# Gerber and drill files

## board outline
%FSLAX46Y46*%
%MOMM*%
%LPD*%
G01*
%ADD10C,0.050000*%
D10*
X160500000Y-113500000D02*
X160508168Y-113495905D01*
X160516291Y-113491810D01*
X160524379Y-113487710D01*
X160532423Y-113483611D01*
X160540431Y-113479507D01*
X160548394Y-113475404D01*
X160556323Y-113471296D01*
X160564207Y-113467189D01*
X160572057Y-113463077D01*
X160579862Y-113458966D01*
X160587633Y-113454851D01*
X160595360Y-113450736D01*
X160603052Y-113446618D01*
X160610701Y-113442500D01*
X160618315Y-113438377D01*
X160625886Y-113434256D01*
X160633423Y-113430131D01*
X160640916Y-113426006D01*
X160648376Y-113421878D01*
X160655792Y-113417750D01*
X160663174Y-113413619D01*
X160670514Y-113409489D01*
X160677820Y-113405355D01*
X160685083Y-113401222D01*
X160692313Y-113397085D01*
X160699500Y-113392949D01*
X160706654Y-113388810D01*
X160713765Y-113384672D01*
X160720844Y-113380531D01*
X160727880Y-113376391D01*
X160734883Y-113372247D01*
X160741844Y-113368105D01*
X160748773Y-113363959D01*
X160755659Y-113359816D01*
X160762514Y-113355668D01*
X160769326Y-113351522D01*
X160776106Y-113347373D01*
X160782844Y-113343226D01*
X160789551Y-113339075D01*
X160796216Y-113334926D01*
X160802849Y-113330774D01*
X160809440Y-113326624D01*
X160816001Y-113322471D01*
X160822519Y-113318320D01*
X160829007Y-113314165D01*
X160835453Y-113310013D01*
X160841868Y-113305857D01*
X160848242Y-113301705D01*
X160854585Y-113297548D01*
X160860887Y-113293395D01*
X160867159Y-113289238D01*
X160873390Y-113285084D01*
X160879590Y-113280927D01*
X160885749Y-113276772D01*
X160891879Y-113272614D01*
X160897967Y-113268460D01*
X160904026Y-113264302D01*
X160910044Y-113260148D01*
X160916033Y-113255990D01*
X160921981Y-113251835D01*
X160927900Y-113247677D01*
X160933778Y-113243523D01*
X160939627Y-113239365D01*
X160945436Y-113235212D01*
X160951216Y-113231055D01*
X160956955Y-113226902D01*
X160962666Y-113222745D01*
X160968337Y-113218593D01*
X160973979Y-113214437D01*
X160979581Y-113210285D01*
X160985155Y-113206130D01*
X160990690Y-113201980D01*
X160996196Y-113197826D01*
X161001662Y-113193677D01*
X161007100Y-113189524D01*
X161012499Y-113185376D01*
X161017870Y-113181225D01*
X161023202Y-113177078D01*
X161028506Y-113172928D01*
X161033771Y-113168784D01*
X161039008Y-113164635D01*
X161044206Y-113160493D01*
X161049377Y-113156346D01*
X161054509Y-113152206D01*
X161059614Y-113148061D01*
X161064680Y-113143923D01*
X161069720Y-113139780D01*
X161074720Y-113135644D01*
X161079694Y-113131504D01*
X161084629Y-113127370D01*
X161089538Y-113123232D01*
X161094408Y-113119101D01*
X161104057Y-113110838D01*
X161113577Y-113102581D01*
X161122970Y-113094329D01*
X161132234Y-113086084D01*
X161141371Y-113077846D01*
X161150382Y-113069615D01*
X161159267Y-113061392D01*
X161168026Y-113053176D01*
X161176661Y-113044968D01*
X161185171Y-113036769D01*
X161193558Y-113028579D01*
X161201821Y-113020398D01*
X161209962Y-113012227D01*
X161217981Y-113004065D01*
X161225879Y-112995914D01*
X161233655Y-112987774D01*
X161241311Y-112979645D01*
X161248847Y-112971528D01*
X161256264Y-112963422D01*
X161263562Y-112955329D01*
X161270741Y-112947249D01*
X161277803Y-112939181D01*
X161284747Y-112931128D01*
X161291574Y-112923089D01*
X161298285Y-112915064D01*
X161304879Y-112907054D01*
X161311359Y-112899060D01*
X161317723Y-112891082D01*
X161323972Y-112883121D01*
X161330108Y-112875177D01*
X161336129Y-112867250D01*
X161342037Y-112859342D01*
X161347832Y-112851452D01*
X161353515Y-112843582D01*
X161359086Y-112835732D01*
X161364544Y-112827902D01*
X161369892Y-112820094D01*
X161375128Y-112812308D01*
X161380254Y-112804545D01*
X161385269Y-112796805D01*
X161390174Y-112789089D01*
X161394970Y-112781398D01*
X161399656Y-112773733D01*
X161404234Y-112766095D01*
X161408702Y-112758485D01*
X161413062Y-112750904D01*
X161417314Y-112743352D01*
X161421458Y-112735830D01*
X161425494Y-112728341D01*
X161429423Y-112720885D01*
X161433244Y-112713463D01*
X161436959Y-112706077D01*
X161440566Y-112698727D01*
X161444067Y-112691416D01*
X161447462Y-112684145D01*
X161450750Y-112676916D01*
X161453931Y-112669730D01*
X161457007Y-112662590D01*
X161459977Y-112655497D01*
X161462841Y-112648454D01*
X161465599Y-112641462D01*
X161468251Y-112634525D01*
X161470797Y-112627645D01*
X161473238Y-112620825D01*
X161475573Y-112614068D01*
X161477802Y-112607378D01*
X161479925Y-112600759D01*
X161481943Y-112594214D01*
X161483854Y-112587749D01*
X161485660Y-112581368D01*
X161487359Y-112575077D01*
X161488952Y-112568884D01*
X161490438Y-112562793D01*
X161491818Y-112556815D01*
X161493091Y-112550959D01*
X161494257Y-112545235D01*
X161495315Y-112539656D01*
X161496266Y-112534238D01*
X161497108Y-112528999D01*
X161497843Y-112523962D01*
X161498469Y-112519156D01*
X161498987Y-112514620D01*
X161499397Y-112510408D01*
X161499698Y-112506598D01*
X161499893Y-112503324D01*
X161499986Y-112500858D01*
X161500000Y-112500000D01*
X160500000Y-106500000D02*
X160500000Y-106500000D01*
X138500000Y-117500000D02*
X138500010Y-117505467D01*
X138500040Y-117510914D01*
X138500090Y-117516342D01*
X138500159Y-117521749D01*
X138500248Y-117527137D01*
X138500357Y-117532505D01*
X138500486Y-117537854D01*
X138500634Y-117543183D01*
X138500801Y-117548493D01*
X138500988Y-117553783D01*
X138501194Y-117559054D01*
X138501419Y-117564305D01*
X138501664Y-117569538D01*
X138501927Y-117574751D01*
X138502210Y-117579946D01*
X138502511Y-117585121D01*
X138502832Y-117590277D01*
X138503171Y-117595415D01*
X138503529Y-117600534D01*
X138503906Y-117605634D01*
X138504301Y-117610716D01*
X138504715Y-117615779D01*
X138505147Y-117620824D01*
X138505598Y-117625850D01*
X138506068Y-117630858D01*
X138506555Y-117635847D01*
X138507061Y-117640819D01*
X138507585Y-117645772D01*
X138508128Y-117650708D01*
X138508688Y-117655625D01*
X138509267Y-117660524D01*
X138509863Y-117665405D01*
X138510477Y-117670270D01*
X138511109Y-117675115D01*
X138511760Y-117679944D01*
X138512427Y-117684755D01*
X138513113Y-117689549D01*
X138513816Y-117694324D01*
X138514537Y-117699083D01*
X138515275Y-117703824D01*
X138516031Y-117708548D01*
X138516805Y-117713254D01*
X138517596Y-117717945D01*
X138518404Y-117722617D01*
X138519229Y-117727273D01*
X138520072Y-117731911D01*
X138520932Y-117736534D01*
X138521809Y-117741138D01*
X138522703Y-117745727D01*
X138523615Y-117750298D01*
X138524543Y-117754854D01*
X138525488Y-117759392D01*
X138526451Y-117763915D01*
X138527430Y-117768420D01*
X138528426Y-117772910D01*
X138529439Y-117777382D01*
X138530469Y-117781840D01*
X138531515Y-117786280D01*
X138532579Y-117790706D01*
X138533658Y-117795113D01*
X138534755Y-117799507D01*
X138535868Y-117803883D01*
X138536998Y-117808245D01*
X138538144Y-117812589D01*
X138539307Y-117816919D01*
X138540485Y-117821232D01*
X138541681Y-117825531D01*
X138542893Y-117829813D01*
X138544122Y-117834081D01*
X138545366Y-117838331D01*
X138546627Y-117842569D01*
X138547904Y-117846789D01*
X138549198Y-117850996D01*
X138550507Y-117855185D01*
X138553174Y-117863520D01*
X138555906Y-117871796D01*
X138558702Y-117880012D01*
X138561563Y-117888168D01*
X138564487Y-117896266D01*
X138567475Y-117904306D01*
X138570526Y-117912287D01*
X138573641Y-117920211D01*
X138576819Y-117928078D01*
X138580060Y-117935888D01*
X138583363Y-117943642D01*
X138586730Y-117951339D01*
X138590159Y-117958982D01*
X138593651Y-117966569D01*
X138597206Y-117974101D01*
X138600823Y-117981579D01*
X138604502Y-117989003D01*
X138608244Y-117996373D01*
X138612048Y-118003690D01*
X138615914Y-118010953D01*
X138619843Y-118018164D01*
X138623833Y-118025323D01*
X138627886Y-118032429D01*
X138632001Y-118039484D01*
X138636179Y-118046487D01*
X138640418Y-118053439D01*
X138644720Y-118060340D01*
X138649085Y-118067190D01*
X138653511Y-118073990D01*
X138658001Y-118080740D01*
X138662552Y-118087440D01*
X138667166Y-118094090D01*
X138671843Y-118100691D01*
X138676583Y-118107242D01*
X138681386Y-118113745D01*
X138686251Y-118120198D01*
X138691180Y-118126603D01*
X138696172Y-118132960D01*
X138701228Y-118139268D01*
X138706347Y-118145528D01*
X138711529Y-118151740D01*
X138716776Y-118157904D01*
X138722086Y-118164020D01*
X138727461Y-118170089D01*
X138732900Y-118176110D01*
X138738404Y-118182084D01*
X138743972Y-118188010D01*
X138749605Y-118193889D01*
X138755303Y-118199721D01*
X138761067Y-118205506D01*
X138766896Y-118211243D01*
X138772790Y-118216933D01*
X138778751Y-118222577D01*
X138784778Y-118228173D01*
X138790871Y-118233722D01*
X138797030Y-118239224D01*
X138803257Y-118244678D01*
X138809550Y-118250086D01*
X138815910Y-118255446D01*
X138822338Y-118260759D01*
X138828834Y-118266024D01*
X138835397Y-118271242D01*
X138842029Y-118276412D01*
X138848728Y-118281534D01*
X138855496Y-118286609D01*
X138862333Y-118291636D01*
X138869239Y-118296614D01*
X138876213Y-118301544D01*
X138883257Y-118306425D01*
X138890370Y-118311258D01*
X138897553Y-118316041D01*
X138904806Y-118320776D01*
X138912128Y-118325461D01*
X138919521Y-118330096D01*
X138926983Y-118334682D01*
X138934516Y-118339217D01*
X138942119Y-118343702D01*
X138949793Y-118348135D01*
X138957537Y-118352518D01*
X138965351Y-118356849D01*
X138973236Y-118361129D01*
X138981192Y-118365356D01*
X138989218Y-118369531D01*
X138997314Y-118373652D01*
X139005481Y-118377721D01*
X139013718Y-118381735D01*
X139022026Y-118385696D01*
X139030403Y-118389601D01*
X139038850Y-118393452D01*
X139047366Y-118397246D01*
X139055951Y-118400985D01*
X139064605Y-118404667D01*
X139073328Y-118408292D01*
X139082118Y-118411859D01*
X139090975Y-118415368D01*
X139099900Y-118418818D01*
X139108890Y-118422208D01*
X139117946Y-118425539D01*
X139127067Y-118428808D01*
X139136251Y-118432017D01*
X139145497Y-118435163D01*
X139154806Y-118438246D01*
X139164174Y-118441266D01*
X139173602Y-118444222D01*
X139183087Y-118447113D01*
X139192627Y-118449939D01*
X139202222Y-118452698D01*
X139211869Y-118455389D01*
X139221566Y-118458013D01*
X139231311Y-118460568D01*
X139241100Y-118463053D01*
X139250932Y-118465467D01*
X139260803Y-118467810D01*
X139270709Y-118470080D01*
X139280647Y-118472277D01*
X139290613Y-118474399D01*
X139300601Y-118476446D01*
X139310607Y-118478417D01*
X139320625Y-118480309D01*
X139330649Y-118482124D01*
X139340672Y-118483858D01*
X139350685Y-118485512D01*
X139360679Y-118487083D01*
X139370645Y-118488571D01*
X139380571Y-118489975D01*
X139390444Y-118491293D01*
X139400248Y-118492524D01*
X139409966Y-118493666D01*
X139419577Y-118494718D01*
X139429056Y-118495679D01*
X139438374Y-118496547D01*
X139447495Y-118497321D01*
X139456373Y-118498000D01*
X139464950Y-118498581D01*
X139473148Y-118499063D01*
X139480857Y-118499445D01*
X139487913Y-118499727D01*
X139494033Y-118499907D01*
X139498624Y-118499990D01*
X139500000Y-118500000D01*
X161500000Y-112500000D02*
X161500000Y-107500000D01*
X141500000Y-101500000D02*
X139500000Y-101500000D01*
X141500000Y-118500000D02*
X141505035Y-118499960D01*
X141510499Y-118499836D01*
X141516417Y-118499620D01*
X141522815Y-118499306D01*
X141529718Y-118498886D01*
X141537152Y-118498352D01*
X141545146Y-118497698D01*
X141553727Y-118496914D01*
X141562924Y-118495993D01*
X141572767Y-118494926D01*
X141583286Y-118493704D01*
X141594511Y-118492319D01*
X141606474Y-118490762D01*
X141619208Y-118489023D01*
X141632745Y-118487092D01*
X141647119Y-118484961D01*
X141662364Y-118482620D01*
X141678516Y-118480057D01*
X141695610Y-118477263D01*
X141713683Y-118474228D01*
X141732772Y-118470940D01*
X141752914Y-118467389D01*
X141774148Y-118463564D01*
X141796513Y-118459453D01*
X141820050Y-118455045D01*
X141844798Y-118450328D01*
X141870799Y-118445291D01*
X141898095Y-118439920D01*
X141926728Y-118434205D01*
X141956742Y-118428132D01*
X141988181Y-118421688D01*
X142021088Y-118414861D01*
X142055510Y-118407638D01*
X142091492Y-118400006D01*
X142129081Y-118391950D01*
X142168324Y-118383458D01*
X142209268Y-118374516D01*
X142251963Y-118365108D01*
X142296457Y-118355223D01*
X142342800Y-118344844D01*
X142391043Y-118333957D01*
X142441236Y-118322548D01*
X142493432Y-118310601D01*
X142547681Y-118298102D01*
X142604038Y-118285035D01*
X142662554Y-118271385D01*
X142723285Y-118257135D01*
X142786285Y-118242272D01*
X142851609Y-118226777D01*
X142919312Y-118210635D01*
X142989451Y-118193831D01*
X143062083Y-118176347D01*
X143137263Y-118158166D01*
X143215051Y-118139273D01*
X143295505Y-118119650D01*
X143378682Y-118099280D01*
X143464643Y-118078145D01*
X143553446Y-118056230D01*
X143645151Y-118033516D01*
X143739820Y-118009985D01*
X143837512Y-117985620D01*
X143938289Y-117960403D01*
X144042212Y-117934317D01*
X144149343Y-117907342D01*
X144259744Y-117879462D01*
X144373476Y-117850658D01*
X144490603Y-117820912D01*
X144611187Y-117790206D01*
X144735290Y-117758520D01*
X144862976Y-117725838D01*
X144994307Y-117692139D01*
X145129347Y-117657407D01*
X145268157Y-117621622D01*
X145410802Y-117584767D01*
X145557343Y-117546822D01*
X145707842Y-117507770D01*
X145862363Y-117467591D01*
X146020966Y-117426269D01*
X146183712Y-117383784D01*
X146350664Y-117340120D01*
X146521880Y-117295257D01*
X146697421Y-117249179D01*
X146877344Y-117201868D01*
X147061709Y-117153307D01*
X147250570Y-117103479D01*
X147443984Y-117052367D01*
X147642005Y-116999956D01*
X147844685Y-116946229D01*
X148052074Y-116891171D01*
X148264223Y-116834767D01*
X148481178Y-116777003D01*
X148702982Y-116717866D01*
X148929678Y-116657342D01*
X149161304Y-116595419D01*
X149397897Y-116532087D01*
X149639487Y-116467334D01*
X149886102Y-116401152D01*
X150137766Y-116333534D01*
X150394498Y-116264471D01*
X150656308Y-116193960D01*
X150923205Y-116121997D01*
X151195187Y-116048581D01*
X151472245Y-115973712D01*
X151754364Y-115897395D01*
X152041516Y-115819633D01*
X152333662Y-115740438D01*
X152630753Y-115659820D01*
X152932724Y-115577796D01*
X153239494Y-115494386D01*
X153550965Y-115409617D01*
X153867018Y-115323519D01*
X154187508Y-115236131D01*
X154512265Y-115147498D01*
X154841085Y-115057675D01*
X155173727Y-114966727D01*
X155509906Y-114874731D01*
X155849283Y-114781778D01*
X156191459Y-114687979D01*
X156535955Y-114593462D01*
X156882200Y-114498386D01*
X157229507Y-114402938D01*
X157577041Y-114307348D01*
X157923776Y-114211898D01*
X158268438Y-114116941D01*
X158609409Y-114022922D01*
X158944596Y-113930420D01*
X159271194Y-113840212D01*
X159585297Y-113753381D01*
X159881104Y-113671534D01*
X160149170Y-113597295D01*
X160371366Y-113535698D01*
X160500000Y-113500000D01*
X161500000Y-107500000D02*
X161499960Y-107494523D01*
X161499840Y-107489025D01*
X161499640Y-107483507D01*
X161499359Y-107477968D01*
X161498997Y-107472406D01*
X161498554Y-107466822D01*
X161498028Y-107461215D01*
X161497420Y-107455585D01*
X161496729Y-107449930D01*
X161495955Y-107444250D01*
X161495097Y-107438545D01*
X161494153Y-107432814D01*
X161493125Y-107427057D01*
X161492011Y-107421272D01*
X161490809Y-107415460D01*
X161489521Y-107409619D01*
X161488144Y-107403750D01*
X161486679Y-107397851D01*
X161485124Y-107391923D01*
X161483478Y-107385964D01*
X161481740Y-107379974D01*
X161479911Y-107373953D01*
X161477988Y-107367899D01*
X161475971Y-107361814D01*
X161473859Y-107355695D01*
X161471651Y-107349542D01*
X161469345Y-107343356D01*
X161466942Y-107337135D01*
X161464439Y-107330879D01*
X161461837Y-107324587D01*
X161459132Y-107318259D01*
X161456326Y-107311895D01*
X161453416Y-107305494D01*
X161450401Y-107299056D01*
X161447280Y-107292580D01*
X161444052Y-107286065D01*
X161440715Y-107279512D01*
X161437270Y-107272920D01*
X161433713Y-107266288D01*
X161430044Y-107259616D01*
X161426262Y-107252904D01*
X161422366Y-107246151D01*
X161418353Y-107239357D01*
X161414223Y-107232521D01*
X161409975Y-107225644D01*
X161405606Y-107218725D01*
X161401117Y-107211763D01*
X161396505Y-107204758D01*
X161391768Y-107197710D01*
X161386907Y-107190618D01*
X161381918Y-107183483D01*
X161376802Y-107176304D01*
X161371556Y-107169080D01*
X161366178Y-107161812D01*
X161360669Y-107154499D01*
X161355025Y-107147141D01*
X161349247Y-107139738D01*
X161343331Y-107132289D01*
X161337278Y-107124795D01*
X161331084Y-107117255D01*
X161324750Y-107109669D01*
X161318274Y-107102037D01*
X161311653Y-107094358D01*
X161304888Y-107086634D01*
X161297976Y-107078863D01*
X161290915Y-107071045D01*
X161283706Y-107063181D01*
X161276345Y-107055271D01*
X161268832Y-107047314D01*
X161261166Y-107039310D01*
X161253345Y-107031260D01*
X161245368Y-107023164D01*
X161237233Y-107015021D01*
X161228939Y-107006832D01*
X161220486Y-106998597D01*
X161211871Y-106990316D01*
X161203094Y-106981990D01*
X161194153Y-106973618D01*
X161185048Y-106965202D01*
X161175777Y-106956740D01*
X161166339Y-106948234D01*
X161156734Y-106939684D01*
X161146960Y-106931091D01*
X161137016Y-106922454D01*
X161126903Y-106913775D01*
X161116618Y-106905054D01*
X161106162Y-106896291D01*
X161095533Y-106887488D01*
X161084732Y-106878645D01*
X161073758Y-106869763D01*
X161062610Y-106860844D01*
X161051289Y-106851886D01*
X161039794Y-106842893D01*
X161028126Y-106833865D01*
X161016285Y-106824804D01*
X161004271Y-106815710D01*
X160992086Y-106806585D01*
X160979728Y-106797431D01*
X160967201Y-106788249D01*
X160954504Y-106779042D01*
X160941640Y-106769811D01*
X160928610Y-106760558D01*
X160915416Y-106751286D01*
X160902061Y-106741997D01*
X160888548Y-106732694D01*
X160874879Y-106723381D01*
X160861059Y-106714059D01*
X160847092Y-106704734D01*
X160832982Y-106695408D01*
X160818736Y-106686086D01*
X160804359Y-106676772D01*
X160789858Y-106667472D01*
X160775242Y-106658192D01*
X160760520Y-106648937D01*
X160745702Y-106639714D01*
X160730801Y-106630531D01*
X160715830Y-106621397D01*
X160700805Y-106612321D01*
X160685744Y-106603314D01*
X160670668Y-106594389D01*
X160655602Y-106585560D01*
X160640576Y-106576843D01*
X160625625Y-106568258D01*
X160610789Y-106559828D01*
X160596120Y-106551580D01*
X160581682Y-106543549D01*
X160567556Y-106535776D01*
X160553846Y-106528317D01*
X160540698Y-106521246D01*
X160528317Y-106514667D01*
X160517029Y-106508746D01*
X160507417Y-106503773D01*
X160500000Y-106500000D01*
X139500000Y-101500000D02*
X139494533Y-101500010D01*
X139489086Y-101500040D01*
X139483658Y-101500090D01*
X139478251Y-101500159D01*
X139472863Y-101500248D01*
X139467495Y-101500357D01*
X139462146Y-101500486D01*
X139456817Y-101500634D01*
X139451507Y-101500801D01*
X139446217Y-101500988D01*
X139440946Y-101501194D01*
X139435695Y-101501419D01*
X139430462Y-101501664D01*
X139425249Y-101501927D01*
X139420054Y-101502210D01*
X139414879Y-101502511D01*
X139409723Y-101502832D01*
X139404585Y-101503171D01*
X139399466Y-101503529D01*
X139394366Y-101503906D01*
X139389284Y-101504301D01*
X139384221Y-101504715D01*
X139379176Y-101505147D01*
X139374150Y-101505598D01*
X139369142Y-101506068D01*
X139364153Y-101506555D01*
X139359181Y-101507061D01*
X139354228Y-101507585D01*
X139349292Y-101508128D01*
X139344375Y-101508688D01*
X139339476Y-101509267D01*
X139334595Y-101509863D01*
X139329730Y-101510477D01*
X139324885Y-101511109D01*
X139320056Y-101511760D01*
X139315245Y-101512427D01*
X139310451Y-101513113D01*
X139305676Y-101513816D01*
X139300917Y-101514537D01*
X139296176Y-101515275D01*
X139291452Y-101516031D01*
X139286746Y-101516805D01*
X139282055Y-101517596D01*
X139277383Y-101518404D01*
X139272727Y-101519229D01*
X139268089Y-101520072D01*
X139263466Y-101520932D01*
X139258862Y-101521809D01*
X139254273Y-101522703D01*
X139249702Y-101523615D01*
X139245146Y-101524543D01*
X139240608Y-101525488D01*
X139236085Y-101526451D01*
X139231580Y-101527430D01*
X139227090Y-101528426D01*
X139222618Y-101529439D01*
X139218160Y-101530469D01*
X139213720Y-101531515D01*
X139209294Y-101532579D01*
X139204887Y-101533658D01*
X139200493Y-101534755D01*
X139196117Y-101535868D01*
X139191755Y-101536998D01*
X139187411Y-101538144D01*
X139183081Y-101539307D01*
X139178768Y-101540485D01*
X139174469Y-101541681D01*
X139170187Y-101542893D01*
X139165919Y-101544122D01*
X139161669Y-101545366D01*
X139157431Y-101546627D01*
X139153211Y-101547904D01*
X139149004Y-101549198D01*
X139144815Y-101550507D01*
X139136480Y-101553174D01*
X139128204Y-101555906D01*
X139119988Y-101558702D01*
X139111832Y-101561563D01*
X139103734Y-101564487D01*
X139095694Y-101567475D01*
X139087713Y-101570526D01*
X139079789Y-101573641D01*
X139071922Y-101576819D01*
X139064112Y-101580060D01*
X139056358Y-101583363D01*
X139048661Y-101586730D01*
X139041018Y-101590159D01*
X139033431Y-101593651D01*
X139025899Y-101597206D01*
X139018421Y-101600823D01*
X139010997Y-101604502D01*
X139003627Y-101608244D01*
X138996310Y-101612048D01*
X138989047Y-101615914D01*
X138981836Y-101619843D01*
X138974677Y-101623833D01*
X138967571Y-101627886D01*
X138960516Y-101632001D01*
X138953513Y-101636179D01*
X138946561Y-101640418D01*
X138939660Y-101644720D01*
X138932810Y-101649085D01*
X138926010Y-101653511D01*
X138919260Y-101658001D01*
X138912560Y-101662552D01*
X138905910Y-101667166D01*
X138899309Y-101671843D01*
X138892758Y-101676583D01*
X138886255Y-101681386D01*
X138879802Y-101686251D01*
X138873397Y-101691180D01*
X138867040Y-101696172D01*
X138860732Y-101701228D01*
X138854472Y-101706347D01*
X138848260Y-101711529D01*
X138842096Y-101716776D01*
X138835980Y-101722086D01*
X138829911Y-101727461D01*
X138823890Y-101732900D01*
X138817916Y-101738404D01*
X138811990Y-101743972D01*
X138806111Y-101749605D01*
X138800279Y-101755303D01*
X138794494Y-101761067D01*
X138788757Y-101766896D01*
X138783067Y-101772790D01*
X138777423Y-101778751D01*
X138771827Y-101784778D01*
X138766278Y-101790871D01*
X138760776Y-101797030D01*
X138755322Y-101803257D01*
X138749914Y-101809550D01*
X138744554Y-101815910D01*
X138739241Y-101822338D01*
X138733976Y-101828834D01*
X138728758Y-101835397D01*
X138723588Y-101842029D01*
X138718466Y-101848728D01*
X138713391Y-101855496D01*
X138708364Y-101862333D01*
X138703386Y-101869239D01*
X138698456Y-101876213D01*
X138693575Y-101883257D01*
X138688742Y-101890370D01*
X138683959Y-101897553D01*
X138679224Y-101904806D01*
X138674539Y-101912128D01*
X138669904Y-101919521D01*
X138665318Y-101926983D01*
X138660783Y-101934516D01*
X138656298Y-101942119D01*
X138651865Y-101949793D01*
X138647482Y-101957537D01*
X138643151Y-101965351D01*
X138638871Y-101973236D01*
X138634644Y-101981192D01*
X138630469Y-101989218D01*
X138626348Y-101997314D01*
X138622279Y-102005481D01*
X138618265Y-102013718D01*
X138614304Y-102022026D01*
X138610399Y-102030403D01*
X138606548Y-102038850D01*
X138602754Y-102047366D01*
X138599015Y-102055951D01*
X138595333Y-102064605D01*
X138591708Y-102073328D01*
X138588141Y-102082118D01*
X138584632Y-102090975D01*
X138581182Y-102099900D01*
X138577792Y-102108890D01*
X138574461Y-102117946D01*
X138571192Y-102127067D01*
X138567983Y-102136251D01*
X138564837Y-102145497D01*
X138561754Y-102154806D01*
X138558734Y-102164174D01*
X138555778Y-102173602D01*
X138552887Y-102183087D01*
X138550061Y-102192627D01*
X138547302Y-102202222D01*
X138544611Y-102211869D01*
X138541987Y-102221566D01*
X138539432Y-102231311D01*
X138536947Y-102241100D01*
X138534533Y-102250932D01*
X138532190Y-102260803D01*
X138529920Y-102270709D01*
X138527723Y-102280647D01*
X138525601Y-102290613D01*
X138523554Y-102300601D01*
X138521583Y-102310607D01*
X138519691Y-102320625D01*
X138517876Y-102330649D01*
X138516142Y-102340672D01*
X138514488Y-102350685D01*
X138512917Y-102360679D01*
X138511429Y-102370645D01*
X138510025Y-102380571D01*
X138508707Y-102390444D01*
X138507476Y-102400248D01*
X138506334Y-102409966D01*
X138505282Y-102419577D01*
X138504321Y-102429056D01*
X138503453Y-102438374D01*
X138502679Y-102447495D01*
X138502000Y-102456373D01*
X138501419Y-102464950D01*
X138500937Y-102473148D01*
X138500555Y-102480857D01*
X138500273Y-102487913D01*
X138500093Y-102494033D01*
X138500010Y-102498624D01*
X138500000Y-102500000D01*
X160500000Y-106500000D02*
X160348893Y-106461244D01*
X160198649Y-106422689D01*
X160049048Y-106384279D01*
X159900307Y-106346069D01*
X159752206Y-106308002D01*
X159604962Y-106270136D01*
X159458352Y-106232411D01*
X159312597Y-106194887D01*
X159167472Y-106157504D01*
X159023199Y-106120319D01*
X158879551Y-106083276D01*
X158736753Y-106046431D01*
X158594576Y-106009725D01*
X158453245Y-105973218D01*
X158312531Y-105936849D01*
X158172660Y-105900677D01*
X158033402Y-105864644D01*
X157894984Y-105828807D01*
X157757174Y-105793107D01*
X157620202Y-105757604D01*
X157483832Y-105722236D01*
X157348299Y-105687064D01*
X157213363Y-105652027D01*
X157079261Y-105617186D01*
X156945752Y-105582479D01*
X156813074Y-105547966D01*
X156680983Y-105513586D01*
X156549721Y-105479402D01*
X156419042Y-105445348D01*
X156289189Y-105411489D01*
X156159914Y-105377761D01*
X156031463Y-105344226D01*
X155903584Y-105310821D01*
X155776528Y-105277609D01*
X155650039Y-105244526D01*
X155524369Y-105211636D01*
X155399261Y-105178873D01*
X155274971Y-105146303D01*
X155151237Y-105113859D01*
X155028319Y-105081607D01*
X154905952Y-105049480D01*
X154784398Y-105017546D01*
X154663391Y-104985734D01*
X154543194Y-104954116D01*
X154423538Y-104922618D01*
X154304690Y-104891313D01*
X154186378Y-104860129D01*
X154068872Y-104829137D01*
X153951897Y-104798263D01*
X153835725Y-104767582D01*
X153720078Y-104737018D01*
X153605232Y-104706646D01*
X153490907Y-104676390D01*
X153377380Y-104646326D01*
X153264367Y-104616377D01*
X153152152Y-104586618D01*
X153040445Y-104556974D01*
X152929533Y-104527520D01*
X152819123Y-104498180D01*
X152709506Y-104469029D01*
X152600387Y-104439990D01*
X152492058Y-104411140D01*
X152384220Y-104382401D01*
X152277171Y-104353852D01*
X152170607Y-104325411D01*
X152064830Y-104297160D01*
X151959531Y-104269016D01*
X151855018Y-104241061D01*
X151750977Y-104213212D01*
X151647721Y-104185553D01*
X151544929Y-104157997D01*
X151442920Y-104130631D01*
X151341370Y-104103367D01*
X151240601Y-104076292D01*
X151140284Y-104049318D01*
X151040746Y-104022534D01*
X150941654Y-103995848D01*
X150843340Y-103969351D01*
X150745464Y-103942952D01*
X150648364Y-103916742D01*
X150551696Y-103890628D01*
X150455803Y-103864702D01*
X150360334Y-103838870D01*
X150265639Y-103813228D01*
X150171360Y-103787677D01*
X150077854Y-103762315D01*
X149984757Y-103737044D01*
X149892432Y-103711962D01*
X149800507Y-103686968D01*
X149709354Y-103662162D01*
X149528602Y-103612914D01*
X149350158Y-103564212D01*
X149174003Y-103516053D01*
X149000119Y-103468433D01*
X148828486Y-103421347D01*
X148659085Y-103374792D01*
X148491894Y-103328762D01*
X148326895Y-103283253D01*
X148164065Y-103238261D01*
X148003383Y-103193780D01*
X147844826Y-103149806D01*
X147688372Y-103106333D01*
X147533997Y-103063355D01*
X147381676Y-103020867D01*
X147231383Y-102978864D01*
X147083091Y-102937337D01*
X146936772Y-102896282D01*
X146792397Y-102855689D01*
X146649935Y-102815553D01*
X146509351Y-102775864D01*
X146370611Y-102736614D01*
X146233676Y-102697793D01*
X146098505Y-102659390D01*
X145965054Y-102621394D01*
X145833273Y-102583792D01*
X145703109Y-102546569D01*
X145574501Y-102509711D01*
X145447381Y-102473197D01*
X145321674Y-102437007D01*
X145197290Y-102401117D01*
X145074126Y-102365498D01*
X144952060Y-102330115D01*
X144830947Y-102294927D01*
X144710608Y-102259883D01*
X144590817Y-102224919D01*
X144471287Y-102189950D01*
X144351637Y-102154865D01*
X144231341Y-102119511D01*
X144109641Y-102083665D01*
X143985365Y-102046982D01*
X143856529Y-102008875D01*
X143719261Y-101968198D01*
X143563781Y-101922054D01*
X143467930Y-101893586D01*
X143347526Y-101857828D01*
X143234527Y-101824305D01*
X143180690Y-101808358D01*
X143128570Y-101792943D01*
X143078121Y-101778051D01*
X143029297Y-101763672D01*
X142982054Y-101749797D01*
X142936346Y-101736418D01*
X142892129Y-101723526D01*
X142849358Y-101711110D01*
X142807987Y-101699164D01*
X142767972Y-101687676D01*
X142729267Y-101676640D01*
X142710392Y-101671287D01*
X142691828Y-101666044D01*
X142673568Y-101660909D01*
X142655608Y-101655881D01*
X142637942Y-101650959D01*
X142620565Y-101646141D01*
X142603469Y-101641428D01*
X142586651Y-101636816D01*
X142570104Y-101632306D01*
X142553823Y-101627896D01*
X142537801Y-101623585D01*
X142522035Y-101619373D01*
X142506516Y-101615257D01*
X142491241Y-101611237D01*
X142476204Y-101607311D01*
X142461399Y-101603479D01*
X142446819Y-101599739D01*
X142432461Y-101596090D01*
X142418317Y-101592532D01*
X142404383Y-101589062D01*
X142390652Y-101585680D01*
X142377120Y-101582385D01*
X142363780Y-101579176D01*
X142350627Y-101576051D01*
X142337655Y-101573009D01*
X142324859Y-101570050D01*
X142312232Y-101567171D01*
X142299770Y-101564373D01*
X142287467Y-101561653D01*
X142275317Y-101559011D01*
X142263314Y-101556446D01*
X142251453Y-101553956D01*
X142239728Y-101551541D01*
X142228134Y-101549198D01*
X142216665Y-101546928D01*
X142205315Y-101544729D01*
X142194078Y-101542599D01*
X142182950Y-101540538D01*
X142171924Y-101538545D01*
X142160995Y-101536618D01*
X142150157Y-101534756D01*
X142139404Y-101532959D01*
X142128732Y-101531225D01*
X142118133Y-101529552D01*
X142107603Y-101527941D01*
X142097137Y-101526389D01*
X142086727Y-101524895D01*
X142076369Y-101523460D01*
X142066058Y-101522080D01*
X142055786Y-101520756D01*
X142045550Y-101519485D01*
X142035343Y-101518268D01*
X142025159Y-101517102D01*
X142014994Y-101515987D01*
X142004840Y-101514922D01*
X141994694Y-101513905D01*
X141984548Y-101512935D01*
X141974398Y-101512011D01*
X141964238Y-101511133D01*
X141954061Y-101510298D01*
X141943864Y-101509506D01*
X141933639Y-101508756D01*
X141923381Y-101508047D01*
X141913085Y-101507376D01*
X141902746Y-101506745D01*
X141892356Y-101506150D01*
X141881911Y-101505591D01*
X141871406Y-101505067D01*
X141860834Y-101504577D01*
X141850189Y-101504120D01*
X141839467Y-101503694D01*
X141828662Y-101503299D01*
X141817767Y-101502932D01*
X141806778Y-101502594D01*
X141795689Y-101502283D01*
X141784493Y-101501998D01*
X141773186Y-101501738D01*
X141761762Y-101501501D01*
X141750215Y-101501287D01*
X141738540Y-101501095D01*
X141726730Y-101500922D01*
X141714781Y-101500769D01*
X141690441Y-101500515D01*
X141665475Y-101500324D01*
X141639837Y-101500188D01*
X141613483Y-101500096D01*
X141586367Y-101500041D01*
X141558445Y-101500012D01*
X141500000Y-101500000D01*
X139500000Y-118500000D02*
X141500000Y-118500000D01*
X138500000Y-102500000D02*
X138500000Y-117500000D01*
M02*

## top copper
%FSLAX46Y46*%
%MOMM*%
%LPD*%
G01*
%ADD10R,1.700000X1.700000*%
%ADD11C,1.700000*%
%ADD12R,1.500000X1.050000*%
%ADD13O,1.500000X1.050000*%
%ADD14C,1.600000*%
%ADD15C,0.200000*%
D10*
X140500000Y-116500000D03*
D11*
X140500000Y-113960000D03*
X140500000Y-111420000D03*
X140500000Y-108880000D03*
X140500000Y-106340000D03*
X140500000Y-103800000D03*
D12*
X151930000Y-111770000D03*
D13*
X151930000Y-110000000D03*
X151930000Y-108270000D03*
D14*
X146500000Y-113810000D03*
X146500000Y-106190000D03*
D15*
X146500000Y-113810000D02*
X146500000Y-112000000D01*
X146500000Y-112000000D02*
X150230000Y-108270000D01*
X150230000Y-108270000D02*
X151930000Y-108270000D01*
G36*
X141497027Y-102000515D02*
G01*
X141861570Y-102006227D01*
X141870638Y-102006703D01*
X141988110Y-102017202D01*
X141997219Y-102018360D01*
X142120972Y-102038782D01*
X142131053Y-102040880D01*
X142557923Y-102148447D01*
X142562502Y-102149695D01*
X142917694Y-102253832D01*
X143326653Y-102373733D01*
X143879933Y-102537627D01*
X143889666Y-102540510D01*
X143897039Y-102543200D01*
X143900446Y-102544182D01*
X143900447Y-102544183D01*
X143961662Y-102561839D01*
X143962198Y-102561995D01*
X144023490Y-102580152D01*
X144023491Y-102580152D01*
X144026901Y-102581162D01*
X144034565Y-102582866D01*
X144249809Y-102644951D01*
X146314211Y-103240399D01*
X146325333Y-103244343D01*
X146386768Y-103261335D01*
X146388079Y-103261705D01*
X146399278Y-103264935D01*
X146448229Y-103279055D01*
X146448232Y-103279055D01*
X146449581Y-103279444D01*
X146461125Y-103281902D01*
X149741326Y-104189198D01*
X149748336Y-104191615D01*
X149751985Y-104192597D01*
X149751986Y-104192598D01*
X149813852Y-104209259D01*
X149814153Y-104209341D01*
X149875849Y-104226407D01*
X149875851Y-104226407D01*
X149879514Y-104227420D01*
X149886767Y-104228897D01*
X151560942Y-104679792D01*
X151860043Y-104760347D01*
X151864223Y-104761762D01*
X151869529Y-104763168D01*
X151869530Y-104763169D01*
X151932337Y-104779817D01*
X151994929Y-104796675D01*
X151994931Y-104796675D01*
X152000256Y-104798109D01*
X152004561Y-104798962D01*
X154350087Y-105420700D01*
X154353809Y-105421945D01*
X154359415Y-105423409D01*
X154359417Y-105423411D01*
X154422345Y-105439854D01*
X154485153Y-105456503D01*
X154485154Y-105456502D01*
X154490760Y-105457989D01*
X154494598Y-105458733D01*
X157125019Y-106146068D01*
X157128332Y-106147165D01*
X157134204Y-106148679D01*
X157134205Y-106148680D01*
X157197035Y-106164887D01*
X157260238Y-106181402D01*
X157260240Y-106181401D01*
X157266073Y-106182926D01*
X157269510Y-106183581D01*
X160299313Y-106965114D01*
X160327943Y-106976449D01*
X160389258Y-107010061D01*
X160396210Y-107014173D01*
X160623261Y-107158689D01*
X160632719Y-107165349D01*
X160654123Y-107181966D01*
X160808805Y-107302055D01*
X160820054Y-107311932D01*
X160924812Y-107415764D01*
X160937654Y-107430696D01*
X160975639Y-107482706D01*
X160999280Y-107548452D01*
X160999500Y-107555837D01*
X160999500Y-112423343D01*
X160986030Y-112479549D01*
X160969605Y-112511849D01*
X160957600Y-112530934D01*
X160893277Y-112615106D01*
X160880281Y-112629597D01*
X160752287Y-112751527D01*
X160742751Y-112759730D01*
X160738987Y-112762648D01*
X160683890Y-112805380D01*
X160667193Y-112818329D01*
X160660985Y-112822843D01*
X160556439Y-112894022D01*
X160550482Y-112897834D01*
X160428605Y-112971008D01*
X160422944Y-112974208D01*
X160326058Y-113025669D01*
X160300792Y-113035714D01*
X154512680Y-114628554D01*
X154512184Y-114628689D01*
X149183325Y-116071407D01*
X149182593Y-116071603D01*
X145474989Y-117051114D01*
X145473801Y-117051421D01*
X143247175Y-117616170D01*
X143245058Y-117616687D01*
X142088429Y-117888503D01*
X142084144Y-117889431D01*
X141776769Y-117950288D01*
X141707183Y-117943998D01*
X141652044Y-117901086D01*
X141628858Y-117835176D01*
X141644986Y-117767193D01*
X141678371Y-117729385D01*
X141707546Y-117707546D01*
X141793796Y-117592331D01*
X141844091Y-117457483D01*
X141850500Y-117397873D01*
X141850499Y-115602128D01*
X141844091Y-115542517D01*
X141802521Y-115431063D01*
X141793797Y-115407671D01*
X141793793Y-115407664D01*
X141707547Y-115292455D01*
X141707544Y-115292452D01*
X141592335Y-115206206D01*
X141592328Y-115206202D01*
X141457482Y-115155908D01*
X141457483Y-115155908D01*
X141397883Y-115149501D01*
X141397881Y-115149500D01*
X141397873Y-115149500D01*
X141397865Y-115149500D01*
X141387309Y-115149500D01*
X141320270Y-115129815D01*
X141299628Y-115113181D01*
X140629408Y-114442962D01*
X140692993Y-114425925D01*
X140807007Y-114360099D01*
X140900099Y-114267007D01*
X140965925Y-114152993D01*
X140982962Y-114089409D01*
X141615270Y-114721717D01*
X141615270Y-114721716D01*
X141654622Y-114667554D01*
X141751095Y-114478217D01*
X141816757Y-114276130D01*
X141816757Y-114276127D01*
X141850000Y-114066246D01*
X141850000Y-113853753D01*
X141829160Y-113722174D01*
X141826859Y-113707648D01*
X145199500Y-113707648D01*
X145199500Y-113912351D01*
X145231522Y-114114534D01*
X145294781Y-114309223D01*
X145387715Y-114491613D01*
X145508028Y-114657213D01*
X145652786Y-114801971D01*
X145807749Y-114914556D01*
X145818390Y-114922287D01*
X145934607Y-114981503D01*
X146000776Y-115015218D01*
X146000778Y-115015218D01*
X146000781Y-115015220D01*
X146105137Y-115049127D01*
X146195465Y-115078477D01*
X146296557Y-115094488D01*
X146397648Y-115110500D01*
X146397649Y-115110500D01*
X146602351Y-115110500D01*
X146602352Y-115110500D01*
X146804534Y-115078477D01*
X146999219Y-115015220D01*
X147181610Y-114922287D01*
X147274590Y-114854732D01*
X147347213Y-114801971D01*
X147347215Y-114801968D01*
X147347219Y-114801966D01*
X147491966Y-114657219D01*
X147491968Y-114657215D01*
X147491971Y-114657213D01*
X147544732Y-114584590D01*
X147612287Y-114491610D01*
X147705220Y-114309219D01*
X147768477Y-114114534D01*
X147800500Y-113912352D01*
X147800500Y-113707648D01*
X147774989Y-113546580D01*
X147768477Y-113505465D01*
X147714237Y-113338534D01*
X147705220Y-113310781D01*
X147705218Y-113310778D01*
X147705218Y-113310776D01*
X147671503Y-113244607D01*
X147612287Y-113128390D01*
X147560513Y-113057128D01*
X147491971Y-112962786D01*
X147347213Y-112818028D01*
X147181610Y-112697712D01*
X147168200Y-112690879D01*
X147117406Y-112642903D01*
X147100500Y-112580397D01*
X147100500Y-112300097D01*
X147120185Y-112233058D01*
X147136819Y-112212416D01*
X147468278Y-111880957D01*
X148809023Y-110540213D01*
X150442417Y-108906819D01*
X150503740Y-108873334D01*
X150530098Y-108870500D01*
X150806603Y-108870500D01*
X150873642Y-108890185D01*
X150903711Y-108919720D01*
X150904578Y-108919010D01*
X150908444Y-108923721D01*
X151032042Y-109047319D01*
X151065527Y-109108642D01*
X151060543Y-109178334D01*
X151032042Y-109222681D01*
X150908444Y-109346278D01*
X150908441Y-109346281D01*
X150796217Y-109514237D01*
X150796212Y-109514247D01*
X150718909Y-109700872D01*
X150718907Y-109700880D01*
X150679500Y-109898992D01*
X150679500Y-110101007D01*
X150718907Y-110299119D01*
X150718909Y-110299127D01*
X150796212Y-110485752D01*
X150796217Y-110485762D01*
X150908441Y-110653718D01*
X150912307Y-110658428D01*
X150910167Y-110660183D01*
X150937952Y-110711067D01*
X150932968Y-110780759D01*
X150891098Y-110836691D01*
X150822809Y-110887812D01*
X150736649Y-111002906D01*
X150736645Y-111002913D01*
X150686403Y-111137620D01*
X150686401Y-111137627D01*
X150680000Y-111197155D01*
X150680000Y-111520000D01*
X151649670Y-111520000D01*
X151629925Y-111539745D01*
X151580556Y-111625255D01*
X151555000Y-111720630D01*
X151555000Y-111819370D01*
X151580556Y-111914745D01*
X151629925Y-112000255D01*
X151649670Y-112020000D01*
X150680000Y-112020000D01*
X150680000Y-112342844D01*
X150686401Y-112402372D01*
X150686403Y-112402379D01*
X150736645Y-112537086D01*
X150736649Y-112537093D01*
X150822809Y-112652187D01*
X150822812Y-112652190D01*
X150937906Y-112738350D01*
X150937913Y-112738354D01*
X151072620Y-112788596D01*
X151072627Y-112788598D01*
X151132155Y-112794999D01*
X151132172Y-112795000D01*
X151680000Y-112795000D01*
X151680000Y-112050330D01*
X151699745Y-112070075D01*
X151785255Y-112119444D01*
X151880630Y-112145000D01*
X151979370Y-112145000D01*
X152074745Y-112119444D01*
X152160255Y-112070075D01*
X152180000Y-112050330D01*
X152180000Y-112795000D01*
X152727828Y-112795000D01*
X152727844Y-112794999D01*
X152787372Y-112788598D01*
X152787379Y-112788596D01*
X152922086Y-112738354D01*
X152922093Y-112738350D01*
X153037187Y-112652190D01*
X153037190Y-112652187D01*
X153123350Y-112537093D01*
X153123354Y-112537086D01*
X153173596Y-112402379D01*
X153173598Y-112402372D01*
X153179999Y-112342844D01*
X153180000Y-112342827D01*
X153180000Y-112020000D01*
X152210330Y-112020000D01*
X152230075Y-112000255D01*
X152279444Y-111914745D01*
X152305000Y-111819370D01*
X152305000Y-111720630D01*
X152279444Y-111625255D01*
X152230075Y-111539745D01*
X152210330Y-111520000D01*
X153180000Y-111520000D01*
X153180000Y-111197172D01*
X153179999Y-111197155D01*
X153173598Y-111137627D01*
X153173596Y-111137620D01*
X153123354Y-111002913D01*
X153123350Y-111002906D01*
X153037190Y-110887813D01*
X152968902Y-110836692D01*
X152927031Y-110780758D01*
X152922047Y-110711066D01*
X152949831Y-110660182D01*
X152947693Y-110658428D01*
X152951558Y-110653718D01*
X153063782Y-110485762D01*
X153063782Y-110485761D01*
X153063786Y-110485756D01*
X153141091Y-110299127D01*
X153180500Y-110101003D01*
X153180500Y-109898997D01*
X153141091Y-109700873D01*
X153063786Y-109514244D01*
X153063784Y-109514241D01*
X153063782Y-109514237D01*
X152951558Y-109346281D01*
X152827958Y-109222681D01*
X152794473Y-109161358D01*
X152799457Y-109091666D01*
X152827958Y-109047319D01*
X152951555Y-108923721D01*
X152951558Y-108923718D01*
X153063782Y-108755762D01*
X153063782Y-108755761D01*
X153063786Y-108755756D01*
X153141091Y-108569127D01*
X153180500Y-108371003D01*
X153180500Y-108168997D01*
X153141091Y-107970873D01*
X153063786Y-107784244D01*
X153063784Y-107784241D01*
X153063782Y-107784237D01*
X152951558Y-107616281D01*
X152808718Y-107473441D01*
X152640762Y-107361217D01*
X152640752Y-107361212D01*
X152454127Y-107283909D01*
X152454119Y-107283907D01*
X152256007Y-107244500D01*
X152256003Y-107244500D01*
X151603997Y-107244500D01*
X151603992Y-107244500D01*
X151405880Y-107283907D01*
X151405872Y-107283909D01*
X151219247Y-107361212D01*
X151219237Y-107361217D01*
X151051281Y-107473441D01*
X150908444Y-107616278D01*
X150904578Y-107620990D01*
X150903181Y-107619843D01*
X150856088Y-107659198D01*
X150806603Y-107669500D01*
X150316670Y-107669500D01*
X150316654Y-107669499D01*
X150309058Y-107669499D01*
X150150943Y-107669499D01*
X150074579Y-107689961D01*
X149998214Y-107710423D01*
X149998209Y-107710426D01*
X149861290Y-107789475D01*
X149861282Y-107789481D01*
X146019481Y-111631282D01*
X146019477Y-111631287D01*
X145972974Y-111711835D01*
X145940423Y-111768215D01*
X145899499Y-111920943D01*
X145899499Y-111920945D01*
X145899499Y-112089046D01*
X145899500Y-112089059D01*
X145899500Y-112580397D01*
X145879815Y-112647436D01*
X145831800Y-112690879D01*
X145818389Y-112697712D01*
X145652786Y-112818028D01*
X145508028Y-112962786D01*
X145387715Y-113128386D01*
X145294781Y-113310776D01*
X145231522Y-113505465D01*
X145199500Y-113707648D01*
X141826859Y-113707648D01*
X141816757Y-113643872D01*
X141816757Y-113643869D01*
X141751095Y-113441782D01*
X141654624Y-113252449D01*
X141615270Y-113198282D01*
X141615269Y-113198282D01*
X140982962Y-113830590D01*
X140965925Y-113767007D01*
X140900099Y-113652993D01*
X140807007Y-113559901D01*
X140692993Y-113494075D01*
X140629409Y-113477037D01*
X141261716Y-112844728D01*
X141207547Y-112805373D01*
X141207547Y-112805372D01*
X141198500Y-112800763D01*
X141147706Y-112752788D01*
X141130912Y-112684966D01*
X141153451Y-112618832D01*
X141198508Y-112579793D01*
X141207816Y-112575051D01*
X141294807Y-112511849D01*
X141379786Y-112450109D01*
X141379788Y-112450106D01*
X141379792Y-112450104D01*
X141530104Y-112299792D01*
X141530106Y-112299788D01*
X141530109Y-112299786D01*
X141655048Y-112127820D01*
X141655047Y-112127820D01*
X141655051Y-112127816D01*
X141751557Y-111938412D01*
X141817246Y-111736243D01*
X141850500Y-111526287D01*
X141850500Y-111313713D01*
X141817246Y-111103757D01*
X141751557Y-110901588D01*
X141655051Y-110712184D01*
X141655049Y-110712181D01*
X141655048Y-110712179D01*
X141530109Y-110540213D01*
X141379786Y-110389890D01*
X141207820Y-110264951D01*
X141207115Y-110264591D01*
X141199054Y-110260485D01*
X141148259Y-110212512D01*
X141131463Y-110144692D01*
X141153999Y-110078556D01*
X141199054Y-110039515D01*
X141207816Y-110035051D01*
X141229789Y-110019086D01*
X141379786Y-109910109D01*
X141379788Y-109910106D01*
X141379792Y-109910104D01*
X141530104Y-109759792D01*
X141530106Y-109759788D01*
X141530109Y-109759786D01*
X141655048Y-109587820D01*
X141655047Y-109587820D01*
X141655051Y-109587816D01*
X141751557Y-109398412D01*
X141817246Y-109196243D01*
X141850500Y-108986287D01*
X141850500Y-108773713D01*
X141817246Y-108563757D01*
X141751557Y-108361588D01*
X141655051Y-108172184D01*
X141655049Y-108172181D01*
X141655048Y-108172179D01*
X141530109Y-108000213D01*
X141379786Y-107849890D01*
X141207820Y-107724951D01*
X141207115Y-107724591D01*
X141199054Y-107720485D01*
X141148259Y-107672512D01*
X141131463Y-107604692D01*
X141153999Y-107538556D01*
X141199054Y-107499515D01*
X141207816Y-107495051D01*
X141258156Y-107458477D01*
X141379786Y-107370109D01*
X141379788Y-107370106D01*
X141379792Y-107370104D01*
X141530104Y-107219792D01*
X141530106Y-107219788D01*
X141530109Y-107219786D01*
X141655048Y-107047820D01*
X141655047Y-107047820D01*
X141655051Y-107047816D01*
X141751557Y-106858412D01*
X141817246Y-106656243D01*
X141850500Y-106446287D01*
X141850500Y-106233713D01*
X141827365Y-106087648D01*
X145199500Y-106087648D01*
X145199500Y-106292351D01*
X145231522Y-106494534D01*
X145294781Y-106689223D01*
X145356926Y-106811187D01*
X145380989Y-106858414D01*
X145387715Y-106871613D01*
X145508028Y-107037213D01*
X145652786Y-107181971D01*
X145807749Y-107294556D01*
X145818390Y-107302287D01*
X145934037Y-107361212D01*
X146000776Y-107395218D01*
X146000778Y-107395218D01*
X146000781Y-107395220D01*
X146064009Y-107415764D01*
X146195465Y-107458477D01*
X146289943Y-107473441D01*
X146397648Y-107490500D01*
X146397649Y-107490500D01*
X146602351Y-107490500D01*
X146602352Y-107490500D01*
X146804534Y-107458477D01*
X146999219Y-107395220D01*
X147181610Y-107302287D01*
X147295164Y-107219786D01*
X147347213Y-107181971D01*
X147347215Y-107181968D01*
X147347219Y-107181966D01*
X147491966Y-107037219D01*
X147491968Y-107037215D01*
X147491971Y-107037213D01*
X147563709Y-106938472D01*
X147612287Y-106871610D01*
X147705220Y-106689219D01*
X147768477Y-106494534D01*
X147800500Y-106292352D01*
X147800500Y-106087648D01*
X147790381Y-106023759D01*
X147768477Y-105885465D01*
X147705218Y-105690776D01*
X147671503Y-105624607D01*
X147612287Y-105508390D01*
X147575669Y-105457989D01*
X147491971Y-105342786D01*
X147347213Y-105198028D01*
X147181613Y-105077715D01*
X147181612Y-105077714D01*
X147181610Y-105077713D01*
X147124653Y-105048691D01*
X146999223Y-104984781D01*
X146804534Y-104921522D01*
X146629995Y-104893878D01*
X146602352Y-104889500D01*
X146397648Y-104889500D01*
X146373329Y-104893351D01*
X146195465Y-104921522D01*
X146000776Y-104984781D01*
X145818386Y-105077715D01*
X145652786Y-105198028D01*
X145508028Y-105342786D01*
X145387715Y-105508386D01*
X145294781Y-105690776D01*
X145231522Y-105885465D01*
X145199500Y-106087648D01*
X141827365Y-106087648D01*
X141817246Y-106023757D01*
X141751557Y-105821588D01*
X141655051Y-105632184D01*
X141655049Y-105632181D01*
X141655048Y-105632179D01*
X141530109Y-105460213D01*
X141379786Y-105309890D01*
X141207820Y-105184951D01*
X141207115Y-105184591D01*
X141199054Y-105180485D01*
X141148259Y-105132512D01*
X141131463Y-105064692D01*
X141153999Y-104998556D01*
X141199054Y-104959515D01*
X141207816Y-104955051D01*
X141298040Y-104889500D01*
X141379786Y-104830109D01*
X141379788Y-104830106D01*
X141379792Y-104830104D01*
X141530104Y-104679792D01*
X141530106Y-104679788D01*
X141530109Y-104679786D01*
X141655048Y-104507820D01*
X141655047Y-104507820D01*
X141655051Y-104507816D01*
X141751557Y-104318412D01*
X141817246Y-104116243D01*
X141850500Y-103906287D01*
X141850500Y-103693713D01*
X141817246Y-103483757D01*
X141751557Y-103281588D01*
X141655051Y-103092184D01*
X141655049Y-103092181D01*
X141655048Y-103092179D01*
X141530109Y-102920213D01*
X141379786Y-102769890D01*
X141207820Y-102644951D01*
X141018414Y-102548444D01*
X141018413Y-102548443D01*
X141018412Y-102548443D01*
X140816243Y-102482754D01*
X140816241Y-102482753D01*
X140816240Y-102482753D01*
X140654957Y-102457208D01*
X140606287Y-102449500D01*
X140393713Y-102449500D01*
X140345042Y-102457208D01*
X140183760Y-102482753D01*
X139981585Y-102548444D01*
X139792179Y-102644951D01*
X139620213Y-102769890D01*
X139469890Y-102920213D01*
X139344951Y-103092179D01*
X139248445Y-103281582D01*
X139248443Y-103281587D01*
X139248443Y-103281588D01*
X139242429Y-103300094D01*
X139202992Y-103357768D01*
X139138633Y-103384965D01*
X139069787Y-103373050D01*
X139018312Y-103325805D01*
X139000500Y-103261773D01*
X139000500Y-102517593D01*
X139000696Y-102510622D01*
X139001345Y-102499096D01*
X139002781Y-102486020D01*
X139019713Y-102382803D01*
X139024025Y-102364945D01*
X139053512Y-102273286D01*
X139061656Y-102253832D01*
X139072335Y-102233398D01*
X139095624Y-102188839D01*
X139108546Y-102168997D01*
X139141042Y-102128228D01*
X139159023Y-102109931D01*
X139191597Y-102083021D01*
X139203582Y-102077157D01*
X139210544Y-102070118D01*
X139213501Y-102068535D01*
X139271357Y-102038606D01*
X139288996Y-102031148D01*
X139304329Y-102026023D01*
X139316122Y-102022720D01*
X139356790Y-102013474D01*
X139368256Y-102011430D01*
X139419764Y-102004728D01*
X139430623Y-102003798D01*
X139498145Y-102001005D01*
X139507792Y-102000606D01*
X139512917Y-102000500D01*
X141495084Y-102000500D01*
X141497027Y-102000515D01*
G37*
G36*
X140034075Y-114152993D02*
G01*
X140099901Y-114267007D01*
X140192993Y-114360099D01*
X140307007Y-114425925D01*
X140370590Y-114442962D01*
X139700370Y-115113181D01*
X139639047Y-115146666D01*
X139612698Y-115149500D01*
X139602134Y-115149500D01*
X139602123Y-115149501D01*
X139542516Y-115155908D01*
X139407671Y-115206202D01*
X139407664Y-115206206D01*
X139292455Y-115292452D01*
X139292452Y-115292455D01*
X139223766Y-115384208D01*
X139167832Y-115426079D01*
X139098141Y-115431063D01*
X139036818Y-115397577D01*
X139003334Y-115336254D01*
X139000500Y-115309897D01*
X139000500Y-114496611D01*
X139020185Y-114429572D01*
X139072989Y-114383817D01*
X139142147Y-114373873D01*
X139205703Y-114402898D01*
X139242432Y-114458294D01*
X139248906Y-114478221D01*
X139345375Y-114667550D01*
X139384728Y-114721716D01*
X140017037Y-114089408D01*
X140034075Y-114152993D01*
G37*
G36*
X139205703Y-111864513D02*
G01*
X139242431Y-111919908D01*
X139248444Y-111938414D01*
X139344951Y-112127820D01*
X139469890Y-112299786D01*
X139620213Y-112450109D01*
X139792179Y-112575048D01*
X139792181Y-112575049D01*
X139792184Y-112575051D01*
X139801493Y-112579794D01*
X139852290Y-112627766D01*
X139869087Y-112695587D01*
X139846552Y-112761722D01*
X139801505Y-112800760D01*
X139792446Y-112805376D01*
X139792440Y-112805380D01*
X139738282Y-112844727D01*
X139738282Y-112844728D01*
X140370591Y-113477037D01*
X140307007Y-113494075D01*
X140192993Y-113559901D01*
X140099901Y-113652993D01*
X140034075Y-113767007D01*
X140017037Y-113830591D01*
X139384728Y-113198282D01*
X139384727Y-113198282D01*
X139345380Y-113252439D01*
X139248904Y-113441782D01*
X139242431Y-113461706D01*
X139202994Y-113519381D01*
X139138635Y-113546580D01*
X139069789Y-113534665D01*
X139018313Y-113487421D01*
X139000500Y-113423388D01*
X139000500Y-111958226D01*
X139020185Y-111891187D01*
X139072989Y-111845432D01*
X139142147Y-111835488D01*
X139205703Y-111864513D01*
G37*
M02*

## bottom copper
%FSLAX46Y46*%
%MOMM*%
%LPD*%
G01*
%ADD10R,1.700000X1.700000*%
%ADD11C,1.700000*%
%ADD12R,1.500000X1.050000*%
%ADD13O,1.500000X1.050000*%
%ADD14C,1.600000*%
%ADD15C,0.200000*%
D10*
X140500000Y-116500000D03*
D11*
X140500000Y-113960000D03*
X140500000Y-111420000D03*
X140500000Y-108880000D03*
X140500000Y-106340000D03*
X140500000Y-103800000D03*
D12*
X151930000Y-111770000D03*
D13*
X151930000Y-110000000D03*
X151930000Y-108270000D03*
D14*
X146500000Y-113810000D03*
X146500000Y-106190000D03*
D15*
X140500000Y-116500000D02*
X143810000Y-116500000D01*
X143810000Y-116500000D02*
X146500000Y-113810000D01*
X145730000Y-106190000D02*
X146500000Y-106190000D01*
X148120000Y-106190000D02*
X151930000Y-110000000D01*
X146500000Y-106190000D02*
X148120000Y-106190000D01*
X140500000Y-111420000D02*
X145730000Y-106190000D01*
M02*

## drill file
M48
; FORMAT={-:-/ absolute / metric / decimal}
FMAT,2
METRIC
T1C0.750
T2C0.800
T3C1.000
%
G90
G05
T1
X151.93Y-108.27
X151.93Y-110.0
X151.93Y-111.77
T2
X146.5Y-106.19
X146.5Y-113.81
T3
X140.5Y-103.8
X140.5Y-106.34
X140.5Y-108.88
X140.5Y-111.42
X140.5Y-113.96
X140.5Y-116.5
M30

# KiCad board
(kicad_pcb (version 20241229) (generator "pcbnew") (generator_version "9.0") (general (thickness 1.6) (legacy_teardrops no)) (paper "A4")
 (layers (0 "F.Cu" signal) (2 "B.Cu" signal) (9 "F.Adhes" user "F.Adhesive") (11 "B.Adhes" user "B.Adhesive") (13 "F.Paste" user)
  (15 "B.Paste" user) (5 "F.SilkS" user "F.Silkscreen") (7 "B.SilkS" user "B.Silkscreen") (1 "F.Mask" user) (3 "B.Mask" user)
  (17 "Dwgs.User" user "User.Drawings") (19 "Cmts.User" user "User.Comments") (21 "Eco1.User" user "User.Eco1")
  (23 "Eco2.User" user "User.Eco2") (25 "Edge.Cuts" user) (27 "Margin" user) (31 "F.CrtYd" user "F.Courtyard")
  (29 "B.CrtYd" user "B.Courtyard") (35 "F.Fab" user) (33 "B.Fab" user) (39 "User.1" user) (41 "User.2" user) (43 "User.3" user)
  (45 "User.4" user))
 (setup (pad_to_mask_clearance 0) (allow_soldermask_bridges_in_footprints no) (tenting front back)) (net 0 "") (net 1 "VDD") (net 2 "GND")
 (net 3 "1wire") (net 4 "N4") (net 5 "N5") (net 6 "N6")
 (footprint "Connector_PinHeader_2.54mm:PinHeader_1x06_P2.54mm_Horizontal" (layer "F.Cu") (at 140.5 116.5 180)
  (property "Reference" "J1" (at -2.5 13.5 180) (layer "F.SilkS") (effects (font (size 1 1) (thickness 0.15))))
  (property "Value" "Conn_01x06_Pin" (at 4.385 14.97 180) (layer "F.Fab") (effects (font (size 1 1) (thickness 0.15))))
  (pad "1" thru_hole rect (at 0 0 180) (size 1.7 1.7) (drill 1) (layers "*.Cu" "*.Mask") (remove_unused_layers no) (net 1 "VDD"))
  (pad "2" thru_hole circle (at 0 2.54 180) (size 1.7 1.7) (drill 1) (layers "*.Cu" "*.Mask") (remove_unused_layers no) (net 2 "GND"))
  (pad "3" thru_hole circle (at 0 5.08 180) (size 1.7 1.7) (drill 1) (layers "*.Cu" "*.Mask") (remove_unused_layers no) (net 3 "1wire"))
  (pad "4" thru_hole circle (at 0 7.62 180) (size 1.7 1.7) (drill 1) (layers "*.Cu" "*.Mask") (remove_unused_layers no) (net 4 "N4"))
  (pad "5" thru_hole circle (at 0 10.16 180) (size 1.7 1.7) (drill 1) (layers "*.Cu" "*.Mask") (remove_unused_layers no) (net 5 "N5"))
  (pad "6" thru_hole circle (at 0 12.7 180) (size 1.7 1.7) (drill 1) (layers "*.Cu" "*.Mask") (remove_unused_layers no) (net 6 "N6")))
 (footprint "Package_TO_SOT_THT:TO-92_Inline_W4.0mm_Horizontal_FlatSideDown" (layer "F.Cu") (at 151.93 111.27 90)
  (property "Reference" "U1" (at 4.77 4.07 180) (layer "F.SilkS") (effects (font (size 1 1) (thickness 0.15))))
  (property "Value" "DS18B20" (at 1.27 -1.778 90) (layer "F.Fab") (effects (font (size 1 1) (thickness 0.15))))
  (pad "1" thru_hole rect (at -0.5 0 90) (size 1.05 1.5) (drill 0.75) (layers "*.Cu" "*.Mask") (remove_unused_layers no) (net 2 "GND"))
  (pad "2" thru_hole oval (at 1.27 0 90) (size 1.05 1.5) (drill 0.75) (layers "*.Cu" "*.Mask") (remove_unused_layers no) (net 3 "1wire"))
  (pad "3" thru_hole oval (at 3 0 90) (size 1.05 1.5) (drill 0.75) (layers "*.Cu" "*.Mask") (remove_unused_layers no) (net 1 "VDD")))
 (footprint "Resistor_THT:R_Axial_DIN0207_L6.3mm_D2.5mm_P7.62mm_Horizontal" (layer "F.Cu") (at 146.5 113.81 90)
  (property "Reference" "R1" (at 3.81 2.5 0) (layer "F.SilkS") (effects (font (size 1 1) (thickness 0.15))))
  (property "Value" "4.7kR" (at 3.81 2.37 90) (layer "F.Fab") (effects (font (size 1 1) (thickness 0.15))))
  (pad "1" thru_hole circle (at 0 0 90) (size 1.6 1.6) (drill 0.8) (layers "*.Cu" "*.Mask") (remove_unused_layers no) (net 1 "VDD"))
  (pad "2" thru_hole circle (at 7.62 0 90) (size 1.6 1.6) (drill 0.8) (layers "*.Cu" "*.Mask") (remove_unused_layers no) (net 3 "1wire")))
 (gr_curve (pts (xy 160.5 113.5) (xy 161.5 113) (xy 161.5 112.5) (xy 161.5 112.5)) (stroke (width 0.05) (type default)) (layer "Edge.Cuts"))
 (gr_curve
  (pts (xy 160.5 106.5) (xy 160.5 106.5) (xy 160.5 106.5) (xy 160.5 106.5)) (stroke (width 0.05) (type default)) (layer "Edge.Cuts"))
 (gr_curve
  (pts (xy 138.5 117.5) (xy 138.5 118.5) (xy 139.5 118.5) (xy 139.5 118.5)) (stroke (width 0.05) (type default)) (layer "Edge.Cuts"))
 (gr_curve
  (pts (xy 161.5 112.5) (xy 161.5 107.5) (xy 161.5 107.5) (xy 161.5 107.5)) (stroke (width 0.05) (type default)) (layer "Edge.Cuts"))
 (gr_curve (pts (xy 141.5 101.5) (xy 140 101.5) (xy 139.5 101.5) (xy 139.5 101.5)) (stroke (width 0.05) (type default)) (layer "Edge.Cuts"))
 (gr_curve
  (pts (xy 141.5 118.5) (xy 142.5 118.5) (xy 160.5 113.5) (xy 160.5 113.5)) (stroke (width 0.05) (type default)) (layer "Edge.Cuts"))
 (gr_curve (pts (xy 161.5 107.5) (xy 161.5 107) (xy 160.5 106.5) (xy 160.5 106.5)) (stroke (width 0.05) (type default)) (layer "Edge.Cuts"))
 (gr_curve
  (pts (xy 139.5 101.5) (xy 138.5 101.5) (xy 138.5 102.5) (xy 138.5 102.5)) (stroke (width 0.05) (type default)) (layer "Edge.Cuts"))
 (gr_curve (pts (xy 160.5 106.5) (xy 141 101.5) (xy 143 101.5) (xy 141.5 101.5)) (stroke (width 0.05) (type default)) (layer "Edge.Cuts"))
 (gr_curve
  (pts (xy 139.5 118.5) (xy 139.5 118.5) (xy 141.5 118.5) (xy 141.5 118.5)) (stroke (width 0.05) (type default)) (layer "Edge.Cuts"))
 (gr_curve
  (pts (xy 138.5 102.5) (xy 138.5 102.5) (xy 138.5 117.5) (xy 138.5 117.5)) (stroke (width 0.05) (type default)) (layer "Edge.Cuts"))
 (segment (start 146.5 113.81) (end 146.5 112) (width 0.2) (layer "F.Cu") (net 1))
 (segment (start 146.5 112) (end 150.23 108.27) (width 0.2) (layer "F.Cu") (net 1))
 (segment (start 150.23 108.27) (end 151.93 108.27) (width 0.2) (layer "F.Cu") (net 1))
 (segment (start 140.5 116.5) (end 143.81 116.5) (width 0.2) (layer "B.Cu") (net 1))
 (segment (start 143.81 116.5) (end 146.5 113.81) (width 0.2) (layer "B.Cu") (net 1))
 (segment (start 145.73 106.19) (end 146.5 106.19) (width 0.2) (layer "B.Cu") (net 3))
 (segment (start 148.12 106.19) (end 151.93 110) (width 0.2) (layer "B.Cu") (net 3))
 (segment (start 146.5 106.19) (end 148.12 106.19) (width 0.2) (layer "B.Cu") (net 3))
 (segment (start 140.5 111.42) (end 145.73 106.19) (width 0.2) (layer "B.Cu") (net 3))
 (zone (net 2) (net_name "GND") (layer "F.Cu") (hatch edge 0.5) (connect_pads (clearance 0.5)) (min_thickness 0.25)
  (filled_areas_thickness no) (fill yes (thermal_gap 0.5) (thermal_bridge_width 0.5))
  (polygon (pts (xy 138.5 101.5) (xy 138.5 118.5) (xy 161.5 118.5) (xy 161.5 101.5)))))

